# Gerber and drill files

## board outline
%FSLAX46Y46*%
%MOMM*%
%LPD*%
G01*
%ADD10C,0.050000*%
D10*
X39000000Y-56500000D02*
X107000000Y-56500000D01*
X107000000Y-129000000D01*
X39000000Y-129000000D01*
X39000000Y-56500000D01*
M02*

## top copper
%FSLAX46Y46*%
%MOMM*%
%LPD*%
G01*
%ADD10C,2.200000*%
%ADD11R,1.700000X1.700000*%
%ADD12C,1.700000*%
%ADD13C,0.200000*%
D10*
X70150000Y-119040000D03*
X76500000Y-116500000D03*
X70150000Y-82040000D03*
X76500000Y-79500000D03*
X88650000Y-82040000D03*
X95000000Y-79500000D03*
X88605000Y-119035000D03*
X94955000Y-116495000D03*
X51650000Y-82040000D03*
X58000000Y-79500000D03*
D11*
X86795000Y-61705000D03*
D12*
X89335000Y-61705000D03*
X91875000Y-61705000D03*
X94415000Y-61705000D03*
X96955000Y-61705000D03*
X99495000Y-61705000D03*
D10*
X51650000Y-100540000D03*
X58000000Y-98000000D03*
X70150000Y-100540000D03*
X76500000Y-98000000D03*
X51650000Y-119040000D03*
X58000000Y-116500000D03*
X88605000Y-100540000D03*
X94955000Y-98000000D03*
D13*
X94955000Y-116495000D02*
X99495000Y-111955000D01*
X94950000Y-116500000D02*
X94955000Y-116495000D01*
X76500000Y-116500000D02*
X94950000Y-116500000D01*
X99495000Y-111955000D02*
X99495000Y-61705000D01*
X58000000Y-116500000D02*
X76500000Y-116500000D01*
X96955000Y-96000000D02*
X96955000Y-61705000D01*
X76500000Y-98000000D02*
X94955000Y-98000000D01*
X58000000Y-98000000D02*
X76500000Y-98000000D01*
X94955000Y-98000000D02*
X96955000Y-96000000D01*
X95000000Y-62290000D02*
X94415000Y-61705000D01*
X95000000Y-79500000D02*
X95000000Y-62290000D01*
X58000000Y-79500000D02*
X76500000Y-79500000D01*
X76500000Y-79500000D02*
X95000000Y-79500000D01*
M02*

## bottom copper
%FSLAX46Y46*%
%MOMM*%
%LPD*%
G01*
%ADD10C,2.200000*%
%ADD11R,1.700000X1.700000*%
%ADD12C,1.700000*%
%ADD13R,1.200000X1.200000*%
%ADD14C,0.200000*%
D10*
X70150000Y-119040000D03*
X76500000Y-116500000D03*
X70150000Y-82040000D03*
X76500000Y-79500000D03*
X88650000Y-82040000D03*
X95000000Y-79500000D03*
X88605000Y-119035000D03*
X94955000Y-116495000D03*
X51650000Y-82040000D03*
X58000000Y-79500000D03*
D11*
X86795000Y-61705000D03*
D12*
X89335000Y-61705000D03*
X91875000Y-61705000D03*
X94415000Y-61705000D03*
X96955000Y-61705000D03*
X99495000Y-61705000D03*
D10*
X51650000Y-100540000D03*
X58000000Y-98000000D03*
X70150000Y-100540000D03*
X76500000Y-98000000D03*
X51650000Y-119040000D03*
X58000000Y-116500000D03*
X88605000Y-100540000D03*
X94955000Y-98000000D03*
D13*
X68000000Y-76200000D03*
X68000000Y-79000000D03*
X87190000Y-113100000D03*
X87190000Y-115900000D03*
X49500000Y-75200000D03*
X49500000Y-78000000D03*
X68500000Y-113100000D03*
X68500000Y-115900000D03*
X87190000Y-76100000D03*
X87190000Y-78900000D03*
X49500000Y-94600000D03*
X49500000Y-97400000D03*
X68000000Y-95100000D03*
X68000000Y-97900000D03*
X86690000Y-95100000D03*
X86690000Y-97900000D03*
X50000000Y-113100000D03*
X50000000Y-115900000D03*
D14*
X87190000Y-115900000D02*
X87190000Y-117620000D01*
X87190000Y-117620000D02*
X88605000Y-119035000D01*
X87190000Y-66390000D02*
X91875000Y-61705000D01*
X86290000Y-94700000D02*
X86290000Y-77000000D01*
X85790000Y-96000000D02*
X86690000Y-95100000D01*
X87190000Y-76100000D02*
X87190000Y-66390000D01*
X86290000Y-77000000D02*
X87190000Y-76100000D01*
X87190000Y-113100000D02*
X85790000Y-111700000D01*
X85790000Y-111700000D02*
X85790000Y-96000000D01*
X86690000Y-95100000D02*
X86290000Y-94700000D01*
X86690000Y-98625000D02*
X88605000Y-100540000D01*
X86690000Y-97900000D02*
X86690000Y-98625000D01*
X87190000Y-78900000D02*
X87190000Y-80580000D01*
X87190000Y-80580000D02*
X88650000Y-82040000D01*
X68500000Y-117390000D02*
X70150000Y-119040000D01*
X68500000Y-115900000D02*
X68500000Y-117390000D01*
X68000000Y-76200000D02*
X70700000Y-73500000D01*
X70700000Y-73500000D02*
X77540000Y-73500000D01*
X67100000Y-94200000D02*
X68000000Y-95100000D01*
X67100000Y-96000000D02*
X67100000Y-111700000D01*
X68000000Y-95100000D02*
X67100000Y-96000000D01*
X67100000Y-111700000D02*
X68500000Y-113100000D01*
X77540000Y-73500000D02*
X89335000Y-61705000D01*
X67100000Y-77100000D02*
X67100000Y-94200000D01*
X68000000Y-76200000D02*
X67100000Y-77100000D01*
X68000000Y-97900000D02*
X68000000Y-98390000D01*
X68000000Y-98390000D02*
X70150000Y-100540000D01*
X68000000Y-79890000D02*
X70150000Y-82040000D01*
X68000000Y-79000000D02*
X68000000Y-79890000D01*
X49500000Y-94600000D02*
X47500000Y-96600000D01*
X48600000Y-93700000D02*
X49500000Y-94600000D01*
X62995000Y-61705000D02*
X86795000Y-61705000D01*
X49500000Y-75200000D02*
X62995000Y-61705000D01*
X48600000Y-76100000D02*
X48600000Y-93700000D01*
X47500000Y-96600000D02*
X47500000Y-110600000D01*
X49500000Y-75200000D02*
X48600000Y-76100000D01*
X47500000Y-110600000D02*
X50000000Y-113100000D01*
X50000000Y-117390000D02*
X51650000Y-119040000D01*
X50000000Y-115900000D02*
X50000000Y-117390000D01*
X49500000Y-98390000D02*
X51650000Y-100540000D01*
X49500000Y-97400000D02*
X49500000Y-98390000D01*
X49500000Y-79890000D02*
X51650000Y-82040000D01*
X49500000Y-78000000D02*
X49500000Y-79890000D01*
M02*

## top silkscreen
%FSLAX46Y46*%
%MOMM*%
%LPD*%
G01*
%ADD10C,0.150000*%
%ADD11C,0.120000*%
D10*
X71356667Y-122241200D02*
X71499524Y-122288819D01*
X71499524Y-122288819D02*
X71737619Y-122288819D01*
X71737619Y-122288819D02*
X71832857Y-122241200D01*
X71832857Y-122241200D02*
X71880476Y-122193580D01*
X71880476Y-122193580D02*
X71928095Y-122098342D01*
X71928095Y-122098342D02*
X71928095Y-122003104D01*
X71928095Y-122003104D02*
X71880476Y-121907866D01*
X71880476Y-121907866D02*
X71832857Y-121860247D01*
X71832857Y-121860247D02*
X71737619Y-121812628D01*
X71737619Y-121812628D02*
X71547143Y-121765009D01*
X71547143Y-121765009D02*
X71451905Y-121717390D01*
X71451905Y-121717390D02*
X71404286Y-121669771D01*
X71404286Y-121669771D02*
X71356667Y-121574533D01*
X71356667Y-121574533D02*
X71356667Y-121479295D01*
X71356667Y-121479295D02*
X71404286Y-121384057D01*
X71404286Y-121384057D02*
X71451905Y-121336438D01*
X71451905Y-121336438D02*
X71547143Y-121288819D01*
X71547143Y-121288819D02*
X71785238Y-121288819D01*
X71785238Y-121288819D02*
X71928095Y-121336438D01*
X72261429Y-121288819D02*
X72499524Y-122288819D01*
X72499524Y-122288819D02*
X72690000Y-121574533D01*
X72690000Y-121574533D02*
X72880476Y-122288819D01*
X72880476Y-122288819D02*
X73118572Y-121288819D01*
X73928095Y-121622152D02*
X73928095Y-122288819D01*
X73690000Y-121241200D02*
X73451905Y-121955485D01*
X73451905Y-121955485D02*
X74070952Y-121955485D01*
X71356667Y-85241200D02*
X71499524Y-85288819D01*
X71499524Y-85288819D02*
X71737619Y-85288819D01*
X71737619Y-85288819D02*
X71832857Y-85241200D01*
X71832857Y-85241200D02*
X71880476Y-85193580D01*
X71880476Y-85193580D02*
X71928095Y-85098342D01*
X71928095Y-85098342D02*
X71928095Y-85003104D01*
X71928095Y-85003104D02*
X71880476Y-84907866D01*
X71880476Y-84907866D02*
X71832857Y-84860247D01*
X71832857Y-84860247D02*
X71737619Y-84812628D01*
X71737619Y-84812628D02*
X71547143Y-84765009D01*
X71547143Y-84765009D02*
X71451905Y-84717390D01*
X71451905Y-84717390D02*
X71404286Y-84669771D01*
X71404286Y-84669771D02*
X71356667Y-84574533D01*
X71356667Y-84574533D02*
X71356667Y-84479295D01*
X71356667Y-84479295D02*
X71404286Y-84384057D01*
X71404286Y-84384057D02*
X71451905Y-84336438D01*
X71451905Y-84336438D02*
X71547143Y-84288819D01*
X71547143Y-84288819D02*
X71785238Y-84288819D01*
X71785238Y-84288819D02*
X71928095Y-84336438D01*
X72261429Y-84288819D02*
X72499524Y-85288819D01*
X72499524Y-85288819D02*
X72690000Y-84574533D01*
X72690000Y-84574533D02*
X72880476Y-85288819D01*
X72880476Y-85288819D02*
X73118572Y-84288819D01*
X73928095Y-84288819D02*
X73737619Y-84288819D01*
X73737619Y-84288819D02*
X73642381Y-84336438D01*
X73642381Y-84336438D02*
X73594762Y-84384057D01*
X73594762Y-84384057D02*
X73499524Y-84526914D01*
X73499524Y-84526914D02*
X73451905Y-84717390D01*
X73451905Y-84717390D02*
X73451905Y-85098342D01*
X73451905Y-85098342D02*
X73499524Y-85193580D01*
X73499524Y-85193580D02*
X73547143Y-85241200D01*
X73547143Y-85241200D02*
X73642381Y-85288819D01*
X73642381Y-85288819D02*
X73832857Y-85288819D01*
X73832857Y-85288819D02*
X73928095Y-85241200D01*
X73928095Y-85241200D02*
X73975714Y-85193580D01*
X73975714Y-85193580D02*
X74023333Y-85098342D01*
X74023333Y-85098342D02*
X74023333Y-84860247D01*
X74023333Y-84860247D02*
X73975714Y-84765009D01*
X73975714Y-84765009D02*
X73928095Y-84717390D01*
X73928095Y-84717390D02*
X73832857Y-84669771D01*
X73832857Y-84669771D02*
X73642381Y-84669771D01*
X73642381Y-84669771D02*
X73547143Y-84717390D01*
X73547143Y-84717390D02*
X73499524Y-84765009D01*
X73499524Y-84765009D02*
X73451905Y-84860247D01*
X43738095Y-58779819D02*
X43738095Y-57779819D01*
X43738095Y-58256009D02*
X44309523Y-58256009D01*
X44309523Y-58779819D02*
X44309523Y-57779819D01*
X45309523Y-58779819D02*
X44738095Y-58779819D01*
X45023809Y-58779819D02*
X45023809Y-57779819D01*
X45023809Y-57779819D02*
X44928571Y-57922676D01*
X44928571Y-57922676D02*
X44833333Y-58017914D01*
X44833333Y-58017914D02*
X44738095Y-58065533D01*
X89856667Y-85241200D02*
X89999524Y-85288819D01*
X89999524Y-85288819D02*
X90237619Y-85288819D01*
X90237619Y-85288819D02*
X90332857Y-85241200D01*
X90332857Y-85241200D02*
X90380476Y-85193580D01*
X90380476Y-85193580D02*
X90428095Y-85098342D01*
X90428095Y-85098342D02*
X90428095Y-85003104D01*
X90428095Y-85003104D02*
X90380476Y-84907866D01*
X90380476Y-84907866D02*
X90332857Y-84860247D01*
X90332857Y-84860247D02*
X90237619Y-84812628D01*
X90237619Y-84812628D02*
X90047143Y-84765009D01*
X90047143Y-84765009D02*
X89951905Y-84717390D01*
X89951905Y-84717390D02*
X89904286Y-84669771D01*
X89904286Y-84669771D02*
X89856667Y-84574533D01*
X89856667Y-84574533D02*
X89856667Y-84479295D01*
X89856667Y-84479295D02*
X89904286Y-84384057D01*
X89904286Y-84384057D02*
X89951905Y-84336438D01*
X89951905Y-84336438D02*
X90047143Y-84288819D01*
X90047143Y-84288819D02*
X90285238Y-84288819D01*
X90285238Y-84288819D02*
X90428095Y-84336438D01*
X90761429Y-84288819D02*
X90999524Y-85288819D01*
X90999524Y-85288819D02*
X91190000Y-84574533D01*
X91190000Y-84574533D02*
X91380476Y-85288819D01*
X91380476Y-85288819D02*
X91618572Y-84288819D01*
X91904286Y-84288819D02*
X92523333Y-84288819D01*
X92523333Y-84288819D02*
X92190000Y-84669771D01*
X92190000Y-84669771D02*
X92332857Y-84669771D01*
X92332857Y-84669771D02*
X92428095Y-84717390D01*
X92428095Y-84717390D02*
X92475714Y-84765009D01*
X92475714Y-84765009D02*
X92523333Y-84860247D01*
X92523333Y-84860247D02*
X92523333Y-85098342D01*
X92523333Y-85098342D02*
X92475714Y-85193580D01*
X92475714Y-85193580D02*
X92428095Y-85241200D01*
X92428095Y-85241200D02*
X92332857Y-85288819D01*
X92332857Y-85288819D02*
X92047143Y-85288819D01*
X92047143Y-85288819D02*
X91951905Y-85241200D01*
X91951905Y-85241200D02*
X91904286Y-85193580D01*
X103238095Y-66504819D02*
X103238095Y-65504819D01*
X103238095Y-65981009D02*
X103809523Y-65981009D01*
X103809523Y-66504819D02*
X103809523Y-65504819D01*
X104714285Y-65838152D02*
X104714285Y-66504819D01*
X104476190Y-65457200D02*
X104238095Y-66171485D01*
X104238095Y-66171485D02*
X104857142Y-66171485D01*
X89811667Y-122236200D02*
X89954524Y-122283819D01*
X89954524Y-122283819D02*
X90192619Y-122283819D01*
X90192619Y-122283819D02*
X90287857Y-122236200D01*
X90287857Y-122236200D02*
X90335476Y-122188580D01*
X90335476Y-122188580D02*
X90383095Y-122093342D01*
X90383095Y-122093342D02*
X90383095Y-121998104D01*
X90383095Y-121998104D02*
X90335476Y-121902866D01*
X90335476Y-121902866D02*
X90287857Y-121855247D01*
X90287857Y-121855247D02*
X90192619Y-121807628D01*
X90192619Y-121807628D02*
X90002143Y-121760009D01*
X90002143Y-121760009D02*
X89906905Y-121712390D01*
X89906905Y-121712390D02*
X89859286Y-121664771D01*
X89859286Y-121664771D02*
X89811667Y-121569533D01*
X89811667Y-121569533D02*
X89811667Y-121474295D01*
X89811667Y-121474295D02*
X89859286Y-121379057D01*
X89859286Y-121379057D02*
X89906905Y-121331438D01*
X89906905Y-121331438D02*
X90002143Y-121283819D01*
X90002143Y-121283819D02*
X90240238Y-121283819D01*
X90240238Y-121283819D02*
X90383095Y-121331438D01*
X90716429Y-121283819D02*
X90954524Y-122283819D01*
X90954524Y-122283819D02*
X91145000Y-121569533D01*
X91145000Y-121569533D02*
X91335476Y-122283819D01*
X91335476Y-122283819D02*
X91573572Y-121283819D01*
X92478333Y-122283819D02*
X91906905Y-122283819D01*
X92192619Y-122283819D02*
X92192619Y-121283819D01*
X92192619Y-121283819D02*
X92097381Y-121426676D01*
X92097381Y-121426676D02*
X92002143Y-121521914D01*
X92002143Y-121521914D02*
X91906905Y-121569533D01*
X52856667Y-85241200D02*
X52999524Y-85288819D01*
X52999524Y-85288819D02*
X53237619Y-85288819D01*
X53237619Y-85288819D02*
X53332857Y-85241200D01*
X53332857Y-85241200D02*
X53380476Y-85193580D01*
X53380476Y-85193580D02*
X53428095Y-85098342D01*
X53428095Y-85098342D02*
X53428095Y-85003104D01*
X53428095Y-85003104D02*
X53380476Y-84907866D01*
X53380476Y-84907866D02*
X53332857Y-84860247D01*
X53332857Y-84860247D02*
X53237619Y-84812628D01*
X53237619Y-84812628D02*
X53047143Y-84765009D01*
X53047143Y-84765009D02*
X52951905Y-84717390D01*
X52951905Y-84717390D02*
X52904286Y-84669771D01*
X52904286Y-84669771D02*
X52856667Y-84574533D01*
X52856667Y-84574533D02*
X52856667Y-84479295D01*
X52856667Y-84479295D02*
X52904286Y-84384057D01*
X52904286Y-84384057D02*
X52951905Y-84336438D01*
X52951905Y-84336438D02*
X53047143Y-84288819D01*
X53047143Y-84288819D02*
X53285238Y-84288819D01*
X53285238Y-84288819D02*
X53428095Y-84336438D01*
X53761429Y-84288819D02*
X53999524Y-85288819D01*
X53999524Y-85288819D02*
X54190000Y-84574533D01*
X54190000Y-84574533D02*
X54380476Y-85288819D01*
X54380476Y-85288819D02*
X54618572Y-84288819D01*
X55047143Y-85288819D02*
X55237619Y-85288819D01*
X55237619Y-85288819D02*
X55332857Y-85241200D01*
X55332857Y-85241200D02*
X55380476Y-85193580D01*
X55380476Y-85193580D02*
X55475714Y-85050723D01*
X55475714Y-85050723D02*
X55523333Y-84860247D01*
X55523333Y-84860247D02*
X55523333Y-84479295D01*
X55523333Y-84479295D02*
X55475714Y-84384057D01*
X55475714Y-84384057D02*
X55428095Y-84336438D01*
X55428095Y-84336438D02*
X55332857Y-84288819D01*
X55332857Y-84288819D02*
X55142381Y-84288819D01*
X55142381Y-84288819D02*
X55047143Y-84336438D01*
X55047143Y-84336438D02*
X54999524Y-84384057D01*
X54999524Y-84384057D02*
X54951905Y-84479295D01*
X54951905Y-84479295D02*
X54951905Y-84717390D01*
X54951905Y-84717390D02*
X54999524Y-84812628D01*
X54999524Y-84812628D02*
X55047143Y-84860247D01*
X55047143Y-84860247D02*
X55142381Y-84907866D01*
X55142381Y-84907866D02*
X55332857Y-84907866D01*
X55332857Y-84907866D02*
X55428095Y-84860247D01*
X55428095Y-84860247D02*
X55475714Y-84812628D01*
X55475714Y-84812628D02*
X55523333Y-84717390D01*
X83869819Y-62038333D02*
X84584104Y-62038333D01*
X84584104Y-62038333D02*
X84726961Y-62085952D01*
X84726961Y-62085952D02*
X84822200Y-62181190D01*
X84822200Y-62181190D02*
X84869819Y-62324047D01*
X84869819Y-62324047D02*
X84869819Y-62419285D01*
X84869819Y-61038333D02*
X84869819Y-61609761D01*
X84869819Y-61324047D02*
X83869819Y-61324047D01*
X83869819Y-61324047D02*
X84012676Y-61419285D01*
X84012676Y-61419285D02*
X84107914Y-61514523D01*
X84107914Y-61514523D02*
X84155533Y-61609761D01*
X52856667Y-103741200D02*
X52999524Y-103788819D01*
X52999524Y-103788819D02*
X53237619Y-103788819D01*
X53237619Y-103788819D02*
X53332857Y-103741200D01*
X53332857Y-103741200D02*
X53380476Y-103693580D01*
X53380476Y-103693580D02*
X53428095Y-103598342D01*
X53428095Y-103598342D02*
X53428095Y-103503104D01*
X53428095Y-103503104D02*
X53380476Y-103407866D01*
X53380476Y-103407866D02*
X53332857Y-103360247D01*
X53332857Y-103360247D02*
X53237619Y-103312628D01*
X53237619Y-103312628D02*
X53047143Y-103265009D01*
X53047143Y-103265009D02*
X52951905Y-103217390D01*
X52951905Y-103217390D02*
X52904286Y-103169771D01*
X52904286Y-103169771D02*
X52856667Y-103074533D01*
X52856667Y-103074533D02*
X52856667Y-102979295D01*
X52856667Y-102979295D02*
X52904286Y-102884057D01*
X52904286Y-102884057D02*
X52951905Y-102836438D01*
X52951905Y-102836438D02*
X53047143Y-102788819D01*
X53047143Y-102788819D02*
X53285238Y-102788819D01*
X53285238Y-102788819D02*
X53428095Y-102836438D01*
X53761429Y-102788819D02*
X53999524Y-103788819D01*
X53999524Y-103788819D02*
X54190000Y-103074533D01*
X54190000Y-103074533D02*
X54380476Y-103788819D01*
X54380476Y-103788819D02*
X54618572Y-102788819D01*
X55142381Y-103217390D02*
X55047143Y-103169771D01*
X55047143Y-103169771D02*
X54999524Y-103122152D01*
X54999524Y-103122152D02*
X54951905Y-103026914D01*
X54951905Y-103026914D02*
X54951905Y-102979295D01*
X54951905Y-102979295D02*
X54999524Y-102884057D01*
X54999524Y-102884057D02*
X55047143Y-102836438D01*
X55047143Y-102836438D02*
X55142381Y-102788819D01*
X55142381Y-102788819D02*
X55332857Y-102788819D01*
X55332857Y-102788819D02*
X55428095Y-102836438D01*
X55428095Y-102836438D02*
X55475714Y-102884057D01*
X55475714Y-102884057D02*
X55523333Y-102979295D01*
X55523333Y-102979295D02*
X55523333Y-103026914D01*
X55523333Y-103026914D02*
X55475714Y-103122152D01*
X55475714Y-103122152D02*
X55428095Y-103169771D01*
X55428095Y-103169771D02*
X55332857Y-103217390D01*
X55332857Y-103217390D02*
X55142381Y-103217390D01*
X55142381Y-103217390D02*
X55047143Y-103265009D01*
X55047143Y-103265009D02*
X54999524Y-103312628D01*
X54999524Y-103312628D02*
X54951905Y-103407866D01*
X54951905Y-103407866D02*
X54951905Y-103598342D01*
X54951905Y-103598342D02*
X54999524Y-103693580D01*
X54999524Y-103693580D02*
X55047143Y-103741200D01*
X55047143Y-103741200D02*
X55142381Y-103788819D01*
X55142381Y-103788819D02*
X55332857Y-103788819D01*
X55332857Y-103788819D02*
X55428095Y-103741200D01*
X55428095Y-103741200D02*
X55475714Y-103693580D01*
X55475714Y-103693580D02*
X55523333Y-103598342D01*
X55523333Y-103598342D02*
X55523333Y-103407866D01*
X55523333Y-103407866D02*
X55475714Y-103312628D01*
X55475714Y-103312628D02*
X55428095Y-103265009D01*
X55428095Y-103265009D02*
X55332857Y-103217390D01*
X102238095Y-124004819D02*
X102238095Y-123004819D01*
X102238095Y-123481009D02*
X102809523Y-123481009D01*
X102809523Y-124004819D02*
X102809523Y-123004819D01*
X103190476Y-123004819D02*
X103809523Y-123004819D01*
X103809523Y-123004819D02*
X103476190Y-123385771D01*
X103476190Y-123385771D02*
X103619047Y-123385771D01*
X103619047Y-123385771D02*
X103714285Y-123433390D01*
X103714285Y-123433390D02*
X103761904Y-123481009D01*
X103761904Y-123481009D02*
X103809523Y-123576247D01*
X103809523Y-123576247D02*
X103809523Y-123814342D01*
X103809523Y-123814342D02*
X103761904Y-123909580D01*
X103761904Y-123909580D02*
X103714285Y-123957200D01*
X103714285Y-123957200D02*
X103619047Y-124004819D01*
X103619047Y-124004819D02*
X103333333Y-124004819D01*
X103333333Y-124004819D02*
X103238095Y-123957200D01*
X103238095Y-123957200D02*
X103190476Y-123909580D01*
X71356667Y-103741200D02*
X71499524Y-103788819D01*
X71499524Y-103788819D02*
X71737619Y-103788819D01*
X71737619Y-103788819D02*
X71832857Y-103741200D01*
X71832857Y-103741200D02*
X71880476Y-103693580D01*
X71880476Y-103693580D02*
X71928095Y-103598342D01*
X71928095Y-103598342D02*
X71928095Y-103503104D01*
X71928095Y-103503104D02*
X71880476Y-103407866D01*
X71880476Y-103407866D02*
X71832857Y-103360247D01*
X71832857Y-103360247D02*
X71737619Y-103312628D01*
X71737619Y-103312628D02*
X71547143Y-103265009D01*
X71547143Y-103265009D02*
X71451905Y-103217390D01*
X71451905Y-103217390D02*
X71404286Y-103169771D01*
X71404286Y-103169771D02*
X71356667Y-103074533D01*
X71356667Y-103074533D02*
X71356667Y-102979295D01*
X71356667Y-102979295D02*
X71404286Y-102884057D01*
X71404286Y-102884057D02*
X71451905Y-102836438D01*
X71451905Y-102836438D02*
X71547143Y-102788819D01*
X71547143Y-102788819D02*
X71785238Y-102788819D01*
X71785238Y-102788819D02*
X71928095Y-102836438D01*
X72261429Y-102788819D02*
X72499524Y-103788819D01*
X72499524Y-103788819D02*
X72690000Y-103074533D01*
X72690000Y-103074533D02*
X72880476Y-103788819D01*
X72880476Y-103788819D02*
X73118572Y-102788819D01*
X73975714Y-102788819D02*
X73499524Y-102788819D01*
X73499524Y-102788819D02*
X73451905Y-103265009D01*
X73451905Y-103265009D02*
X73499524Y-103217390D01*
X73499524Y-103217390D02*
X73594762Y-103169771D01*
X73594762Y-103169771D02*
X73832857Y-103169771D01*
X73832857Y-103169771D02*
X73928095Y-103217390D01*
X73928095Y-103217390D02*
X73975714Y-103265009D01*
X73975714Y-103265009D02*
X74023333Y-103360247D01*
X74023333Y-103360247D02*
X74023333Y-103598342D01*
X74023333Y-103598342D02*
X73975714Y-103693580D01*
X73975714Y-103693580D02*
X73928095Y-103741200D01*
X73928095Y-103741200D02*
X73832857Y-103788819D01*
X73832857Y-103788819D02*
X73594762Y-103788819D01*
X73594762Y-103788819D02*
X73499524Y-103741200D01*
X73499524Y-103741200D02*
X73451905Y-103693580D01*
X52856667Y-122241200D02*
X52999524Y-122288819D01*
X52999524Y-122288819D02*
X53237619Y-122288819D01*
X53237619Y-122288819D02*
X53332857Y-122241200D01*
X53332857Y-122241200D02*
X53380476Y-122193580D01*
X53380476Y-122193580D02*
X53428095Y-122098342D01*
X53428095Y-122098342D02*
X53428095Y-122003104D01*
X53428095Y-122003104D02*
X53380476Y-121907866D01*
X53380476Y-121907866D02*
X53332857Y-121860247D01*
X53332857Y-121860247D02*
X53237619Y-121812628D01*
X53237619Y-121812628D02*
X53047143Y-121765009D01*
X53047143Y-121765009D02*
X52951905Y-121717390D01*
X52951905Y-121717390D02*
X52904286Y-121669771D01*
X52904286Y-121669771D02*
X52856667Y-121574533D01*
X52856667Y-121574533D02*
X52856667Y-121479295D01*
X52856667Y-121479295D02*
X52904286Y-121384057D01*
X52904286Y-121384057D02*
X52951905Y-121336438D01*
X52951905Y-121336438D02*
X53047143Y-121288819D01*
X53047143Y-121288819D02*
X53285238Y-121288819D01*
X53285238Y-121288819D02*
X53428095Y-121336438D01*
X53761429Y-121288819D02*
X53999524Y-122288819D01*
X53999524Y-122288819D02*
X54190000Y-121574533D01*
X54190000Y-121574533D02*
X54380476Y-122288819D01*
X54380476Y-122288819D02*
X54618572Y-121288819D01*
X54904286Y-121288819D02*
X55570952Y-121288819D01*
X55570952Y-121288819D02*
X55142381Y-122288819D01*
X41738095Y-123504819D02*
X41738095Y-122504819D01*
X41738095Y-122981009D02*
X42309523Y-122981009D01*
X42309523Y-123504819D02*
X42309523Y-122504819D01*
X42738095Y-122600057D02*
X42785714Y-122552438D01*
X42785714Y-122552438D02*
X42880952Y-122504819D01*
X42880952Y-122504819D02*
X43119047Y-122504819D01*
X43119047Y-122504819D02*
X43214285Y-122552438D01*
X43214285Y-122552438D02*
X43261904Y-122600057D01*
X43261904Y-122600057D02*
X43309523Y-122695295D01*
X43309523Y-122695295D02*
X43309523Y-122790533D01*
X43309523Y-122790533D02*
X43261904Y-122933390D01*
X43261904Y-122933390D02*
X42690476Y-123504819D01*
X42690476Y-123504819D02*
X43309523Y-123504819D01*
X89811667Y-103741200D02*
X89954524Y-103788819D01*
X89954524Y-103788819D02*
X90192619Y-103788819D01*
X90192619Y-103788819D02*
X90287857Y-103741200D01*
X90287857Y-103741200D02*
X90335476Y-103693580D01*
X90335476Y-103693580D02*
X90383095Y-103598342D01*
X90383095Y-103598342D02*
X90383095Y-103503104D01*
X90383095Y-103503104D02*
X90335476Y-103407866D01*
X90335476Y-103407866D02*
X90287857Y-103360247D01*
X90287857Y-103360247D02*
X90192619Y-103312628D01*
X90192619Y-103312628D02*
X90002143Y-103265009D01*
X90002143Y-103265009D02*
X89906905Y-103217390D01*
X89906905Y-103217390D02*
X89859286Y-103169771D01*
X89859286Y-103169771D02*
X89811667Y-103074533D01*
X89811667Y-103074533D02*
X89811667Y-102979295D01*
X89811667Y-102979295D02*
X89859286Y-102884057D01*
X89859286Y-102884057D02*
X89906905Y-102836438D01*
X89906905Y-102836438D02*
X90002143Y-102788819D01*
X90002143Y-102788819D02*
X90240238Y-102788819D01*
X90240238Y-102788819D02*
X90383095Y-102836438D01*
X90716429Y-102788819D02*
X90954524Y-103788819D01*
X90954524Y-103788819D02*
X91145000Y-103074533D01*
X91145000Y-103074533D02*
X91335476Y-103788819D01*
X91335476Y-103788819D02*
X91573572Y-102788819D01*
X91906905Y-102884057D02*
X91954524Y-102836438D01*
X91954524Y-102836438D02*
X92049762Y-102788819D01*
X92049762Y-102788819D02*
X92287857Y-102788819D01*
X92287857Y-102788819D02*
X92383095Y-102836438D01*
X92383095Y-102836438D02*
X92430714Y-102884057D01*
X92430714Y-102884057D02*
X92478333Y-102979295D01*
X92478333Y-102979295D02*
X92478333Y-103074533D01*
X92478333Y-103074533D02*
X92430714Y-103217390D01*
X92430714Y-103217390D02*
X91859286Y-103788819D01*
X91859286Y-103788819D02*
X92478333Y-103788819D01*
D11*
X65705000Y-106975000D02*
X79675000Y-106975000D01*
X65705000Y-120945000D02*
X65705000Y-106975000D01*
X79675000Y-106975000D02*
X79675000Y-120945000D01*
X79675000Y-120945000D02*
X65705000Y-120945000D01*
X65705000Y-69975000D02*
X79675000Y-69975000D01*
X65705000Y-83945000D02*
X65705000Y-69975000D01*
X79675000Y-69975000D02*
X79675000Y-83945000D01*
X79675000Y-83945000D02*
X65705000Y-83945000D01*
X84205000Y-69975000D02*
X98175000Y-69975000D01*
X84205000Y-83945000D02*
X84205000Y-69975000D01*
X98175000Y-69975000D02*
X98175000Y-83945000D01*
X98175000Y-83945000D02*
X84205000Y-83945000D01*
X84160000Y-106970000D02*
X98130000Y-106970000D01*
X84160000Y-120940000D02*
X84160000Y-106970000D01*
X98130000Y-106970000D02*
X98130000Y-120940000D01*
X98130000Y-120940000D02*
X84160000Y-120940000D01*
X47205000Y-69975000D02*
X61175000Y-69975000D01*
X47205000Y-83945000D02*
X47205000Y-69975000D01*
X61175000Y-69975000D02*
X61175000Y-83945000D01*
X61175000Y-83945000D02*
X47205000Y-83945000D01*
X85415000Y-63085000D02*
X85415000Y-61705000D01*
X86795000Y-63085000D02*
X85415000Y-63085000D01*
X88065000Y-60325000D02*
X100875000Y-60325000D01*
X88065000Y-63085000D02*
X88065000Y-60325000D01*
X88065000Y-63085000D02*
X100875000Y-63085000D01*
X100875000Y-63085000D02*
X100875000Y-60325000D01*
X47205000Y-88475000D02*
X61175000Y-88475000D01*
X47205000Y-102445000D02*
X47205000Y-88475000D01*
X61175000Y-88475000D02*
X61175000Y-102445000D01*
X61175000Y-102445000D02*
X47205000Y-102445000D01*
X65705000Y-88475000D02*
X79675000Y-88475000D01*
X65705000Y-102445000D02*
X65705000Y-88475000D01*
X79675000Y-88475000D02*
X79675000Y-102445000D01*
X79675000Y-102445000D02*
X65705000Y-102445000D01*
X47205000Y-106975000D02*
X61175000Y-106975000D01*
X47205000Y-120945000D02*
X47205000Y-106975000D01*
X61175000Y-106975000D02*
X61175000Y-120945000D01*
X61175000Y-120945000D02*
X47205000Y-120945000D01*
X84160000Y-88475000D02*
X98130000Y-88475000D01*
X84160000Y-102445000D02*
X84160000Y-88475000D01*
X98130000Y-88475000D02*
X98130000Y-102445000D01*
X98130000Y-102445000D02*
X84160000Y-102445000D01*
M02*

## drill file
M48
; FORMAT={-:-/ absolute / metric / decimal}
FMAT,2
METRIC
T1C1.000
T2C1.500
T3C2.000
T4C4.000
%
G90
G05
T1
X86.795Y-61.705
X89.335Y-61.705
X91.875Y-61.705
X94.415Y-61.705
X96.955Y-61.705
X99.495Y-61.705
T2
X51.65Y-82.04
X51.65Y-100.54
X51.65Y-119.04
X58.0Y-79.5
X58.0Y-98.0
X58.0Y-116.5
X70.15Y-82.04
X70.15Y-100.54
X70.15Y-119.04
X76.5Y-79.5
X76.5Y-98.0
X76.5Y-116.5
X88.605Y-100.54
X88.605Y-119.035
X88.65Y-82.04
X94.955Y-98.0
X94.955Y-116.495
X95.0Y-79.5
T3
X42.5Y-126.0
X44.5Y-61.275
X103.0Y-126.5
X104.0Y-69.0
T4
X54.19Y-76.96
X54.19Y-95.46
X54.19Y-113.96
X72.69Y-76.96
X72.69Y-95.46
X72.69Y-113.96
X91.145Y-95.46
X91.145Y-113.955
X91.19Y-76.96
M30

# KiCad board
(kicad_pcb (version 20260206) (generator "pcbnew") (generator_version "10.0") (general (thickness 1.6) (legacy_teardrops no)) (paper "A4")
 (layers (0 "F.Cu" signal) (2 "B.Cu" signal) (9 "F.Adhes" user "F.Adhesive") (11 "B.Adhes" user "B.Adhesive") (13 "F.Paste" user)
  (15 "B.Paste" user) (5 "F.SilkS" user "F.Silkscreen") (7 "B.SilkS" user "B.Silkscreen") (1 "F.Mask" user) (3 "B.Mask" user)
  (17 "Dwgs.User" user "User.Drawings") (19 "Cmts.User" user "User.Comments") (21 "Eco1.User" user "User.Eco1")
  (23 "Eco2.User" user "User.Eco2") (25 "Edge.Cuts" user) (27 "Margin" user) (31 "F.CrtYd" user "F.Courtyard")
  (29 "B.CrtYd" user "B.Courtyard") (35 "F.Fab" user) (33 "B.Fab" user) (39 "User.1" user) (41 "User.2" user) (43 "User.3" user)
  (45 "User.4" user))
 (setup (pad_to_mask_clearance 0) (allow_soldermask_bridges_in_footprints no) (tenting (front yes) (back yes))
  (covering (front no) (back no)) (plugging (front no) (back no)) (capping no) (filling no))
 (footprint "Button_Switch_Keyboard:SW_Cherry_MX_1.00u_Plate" (layer "F.Cu") (at 70.15 119.04 180)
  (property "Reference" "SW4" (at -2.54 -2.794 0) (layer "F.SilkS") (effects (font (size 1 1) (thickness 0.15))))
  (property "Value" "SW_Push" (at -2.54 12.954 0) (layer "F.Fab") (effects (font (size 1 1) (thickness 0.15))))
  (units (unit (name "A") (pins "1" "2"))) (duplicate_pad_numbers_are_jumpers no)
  (fp_line (start 4.445 12.065) (end -9.525 12.065) (stroke (width 0.12) (type solid)) (layer "F.SilkS"))
  (fp_line (start 4.445 -1.905) (end 4.445 12.065) (stroke (width 0.12) (type solid)) (layer "F.SilkS"))
  (fp_line (start -9.525 12.065) (end -9.525 -1.905) (stroke (width 0.12) (type solid)) (layer "F.SilkS"))
  (fp_line (start -9.525 -1.905) (end 4.445 -1.905) (stroke (width 0.12) (type solid)) (layer "F.SilkS"))
  (pad "" np_thru_hole circle (at -2.54 5.08 180) (size 4 4) (drill 4) (layers "*.Cu" "*.Mask"))
  (pad "1" thru_hole circle (at 0 0 180) (size 2.2 2.2) (drill 1.5) (layers "*.Cu" "*.Mask") (remove_unused_layers no) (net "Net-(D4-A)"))
  (pad "2" thru_hole circle (at -6.35 2.54 180) (size 2.2 2.2) (drill 1.5) (layers "*.Cu" "*.Mask") (remove_unused_layers no) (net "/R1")))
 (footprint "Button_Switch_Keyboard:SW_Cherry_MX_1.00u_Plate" (layer "F.Cu") (at 70.15 82.04 180)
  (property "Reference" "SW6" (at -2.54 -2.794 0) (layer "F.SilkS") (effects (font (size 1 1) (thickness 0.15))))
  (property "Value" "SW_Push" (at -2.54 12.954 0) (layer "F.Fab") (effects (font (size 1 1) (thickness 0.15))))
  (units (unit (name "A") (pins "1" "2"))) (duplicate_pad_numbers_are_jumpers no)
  (fp_line (start 4.445 12.065) (end -9.525 12.065) (stroke (width 0.12) (type solid)) (layer "F.SilkS"))
  (fp_line (start 4.445 -1.905) (end 4.445 12.065) (stroke (width 0.12) (type solid)) (layer "F.SilkS"))
  (fp_line (start -9.525 12.065) (end -9.525 -1.905) (stroke (width 0.12) (type solid)) (layer "F.SilkS"))
  (fp_line (start -9.525 -1.905) (end 4.445 -1.905) (stroke (width 0.12) (type solid)) (layer "F.SilkS"))
  (pad "" np_thru_hole circle (at -2.54 5.08 180) (size 4 4) (drill 4) (layers "*.Cu" "*.Mask"))
  (pad "1" thru_hole circle (at 0 0 180) (size 2.2 2.2) (drill 1.5) (layers "*.Cu" "*.Mask") (remove_unused_layers no) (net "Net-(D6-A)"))
  (pad "2" thru_hole circle (at -6.35 2.54 180) (size 2.2 2.2) (drill 1.5) (layers "*.Cu" "*.Mask") (remove_unused_layers no) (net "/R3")))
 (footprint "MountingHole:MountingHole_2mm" (layer "F.Cu") (at 44.5 61.275)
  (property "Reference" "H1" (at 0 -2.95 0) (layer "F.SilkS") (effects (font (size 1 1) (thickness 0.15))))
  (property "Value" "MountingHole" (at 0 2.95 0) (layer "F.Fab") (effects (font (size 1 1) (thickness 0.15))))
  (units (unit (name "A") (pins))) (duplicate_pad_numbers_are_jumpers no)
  (pad "" np_thru_hole circle (at 0 0) (size 2 2) (drill 2) (layers "*.Cu" "*.Mask")))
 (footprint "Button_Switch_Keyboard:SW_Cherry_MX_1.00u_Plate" (layer "F.Cu") (at 88.65 82.04 180)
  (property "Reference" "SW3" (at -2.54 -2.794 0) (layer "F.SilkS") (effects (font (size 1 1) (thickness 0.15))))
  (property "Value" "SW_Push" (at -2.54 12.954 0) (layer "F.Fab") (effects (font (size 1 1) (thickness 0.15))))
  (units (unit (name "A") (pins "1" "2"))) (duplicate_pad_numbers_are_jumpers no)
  (fp_line (start 4.445 12.065) (end -9.525 12.065) (stroke (width 0.12) (type solid)) (layer "F.SilkS"))
  (fp_line (start 4.445 -1.905) (end 4.445 12.065) (stroke (width 0.12) (type solid)) (layer "F.SilkS"))
  (fp_line (start -9.525 12.065) (end -9.525 -1.905) (stroke (width 0.12) (type solid)) (layer "F.SilkS"))
  (fp_line (start -9.525 -1.905) (end 4.445 -1.905) (stroke (width 0.12) (type solid)) (layer "F.SilkS"))
  (pad "" np_thru_hole circle (at -2.54 5.08 180) (size 4 4) (drill 4) (layers "*.Cu" "*.Mask"))
  (pad "1" thru_hole circle (at 0 0 180) (size 2.2 2.2) (drill 1.5) (layers "*.Cu" "*.Mask") (remove_unused_layers no) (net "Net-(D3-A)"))
  (pad "2" thru_hole circle (at -6.35 2.54 180) (size 2.2 2.2) (drill 1.5) (layers "*.Cu" "*.Mask") (remove_unused_layers no) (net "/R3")))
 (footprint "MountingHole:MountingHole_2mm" (layer "F.Cu") (at 104 69)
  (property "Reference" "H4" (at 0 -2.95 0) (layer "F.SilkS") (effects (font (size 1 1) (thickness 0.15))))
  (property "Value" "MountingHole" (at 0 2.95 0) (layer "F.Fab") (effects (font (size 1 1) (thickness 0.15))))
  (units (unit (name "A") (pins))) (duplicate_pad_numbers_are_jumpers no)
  (pad "" np_thru_hole circle (at 0 0) (size 2 2) (drill 2) (layers "*.Cu" "*.Mask")))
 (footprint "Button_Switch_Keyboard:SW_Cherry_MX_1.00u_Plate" (layer "F.Cu") (at 88.605 119.035 180)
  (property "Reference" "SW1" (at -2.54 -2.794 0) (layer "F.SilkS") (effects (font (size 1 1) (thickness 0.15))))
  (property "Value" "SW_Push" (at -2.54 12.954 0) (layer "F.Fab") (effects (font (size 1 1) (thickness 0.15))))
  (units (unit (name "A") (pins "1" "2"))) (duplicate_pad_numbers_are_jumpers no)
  (fp_line (start 4.445 12.065) (end -9.525 12.065) (stroke (width 0.12) (type solid)) (layer "F.SilkS"))
  (fp_line (start 4.445 -1.905) (end 4.445 12.065) (stroke (width 0.12) (type solid)) (layer "F.SilkS"))
  (fp_line (start -9.525 12.065) (end -9.525 -1.905) (stroke (width 0.12) (type solid)) (layer "F.SilkS"))
  (fp_line (start -9.525 -1.905) (end 4.445 -1.905) (stroke (width 0.12) (type solid)) (layer "F.SilkS"))
  (pad "" np_thru_hole circle (at -2.54 5.08 180) (size 4 4) (drill 4) (layers "*.Cu" "*.Mask"))
  (pad "1" thru_hole circle (at 0 0 180) (size 2.2 2.2) (drill 1.5) (layers "*.Cu" "*.Mask") (remove_unused_layers no) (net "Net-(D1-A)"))
  (pad "2" thru_hole circle (at -6.35 2.54 180) (size 2.2 2.2) (drill 1.5) (layers "*.Cu" "*.Mask") (remove_unused_layers no) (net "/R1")))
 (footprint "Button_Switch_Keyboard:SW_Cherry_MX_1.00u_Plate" (layer "F.Cu") (at 51.65 82.04 180)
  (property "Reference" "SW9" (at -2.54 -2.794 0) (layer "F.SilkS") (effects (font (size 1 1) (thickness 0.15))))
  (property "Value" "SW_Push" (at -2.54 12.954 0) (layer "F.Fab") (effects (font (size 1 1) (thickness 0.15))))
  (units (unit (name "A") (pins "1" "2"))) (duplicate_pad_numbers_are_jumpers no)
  (fp_line (start 4.445 12.065) (end -9.525 12.065) (stroke (width 0.12) (type solid)) (layer "F.SilkS"))
  (fp_line (start 4.445 -1.905) (end 4.445 12.065) (stroke (width 0.12) (type solid)) (layer "F.SilkS"))
  (fp_line (start -9.525 12.065) (end -9.525 -1.905) (stroke (width 0.12) (type solid)) (layer "F.SilkS"))
  (fp_line (start -9.525 -1.905) (end 4.445 -1.905) (stroke (width 0.12) (type solid)) (layer "F.SilkS"))
  (pad "" np_thru_hole circle (at -2.54 5.08 180) (size 4 4) (drill 4) (layers "*.Cu" "*.Mask"))
  (pad "1" thru_hole circle (at 0 0 180) (size 2.2 2.2) (drill 1.5) (layers "*.Cu" "*.Mask") (remove_unused_layers no) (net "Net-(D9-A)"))
  (pad "2" thru_hole circle (at -6.35 2.54 180) (size 2.2 2.2) (drill 1.5) (layers "*.Cu" "*.Mask") (remove_unused_layers no) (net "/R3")))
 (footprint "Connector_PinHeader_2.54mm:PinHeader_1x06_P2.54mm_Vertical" (layer "F.Cu") (at 86.795 61.705 90)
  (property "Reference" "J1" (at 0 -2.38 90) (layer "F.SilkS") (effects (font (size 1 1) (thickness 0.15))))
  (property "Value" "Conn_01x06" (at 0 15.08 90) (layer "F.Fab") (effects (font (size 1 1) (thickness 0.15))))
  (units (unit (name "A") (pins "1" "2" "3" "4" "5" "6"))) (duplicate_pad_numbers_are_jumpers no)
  (fp_line (start -1.38 -1.38) (end 0 -1.38) (stroke (width 0.12) (type solid)) (layer "F.SilkS"))
  (fp_line (start -1.38 0) (end -1.38 -1.38) (stroke (width 0.12) (type solid)) (layer "F.SilkS"))
  (fp_line (start 1.38 1.27) (end 1.38 14.08) (stroke (width 0.12) (type solid)) (layer "F.SilkS"))
  (fp_line (start -1.38 1.27) (end 1.38 1.27) (stroke (width 0.12) (type solid)) (layer "F.SilkS"))
  (fp_line (start -1.38 1.27) (end -1.38 14.08) (stroke (width 0.12) (type solid)) (layer "F.SilkS"))
  (fp_line (start -1.38 14.08) (end 1.38 14.08) (stroke (width 0.12) (type solid)) (layer "F.SilkS"))
  (pad "1" thru_hole rect (at 0 0 90) (size 1.7 1.7) (drill 1) (layers "*.Cu" "*.Mask") (remove_unused_layers no) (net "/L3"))
  (pad "2" thru_hole circle (at 0 2.54 90) (size 1.7 1.7) (drill 1) (layers "*.Cu" "*.Mask") (remove_unused_layers no) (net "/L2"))
  (pad "3" thru_hole circle (at 0 5.08 90) (size 1.7 1.7) (drill 1) (layers "*.Cu" "*.Mask") (remove_unused_layers no) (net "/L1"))
  (pad "4" thru_hole circle (at 0 7.62 90) (size 1.7 1.7) (drill 1) (layers "*.Cu" "*.Mask") (remove_unused_layers no) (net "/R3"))
  (pad "5" thru_hole circle (at 0 10.16 90) (size 1.7 1.7) (drill 1) (layers "*.Cu" "*.Mask") (remove_unused_layers no) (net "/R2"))
  (pad "6" thru_hole circle (at 0 12.7 90) (size 1.7 1.7) (drill 1) (layers "*.Cu" "*.Mask") (remove_unused_layers no) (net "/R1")))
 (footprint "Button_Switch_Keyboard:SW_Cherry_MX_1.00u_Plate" (layer "F.Cu") (at 51.65 100.54 180)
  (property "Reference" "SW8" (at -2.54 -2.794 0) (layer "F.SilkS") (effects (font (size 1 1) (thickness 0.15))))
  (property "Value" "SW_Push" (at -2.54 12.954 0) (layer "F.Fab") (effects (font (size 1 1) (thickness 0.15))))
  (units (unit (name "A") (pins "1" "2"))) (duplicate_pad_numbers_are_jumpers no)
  (fp_line (start 4.445 12.065) (end -9.525 12.065) (stroke (width 0.12) (type solid)) (layer "F.SilkS"))
  (fp_line (start 4.445 -1.905) (end 4.445 12.065) (stroke (width 0.12) (type solid)) (layer "F.SilkS"))
  (fp_line (start -9.525 12.065) (end -9.525 -1.905) (stroke (width 0.12) (type solid)) (layer "F.SilkS"))
  (fp_line (start -9.525 -1.905) (end 4.445 -1.905) (stroke (width 0.12) (type solid)) (layer "F.SilkS"))
  (pad "" np_thru_hole circle (at -2.54 5.08 180) (size 4 4) (drill 4) (layers "*.Cu" "*.Mask"))
  (pad "1" thru_hole circle (at 0 0 180) (size 2.2 2.2) (drill 1.5) (layers "*.Cu" "*.Mask") (remove_unused_layers no) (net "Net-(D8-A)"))
  (pad "2" thru_hole circle (at -6.35 2.54 180) (size 2.2 2.2) (drill 1.5) (layers "*.Cu" "*.Mask") (remove_unused_layers no) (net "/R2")))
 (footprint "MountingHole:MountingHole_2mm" (layer "F.Cu") (at 103 126.5)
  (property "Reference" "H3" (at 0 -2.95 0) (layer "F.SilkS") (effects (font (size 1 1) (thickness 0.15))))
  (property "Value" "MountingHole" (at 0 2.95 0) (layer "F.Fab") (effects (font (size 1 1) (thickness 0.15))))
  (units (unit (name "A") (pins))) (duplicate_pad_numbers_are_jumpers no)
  (pad "" np_thru_hole circle (at 0 0) (size 2 2) (drill 2) (layers "*.Cu" "*.Mask")))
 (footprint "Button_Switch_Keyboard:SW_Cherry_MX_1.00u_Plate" (layer "F.Cu") (at 70.15 100.54 180)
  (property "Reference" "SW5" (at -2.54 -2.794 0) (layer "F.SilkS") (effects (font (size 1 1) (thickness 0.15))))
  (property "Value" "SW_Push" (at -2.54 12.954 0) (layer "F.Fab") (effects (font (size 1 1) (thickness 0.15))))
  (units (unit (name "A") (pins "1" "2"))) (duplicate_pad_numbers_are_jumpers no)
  (fp_line (start 4.445 12.065) (end -9.525 12.065) (stroke (width 0.12) (type solid)) (layer "F.SilkS"))
  (fp_line (start 4.445 -1.905) (end 4.445 12.065) (stroke (width 0.12) (type solid)) (layer "F.SilkS"))
  (fp_line (start -9.525 12.065) (end -9.525 -1.905) (stroke (width 0.12) (type solid)) (layer "F.SilkS"))
  (fp_line (start -9.525 -1.905) (end 4.445 -1.905) (stroke (width 0.12) (type solid)) (layer "F.SilkS"))
  (pad "" np_thru_hole circle (at -2.54 5.08 180) (size 4 4) (drill 4) (layers "*.Cu" "*.Mask"))
  (pad "1" thru_hole circle (at 0 0 180) (size 2.2 2.2) (drill 1.5) (layers "*.Cu" "*.Mask") (remove_unused_layers no) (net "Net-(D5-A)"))
  (pad "2" thru_hole circle (at -6.35 2.54 180) (size 2.2 2.2) (drill 1.5) (layers "*.Cu" "*.Mask") (remove_unused_layers no) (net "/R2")))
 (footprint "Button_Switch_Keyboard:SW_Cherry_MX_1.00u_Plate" (layer "F.Cu") (at 51.65 119.04 180)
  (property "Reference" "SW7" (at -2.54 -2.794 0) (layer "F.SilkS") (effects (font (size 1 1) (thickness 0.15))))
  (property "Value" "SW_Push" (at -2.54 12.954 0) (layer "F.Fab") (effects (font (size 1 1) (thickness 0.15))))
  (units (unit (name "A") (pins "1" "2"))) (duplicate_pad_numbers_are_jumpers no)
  (fp_line (start 4.445 12.065) (end -9.525 12.065) (stroke (width 0.12) (type solid)) (layer "F.SilkS"))
  (fp_line (start 4.445 -1.905) (end 4.445 12.065) (stroke (width 0.12) (type solid)) (layer "F.SilkS"))
  (fp_line (start -9.525 12.065) (end -9.525 -1.905) (stroke (width 0.12) (type solid)) (layer "F.SilkS"))
  (fp_line (start -9.525 -1.905) (end 4.445 -1.905) (stroke (width 0.12) (type solid)) (layer "F.SilkS"))
  (pad "" np_thru_hole circle (at -2.54 5.08 180) (size 4 4) (drill 4) (layers "*.Cu" "*.Mask"))
  (pad "1" thru_hole circle (at 0 0 180) (size 2.2 2.2) (drill 1.5) (layers "*.Cu" "*.Mask") (remove_unused_layers no) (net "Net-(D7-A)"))
  (pad "2" thru_hole circle (at -6.35 2.54 180) (size 2.2 2.2) (drill 1.5) (layers "*.Cu" "*.Mask") (remove_unused_layers no) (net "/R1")))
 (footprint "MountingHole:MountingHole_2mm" (layer "F.Cu") (at 42.5 126)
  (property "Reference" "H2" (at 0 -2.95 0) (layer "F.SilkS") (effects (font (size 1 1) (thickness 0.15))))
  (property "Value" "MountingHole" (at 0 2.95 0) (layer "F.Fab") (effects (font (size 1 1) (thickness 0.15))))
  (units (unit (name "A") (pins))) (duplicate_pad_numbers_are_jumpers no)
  (pad "" np_thru_hole circle (at 0 0) (size 2 2) (drill 2) (layers "*.Cu" "*.Mask")))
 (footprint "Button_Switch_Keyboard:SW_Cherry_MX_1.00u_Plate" (layer "F.Cu") (at 88.605 100.54 180)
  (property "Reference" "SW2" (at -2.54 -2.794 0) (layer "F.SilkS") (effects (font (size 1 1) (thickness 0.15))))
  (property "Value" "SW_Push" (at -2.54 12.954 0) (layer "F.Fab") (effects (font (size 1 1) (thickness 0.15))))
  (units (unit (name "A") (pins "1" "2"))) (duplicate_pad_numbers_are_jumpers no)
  (fp_line (start 4.445 12.065) (end -9.525 12.065) (stroke (width 0.12) (type solid)) (layer "F.SilkS"))
  (fp_line (start 4.445 -1.905) (end 4.445 12.065) (stroke (width 0.12) (type solid)) (layer "F.SilkS"))
  (fp_line (start -9.525 12.065) (end -9.525 -1.905) (stroke (width 0.12) (type solid)) (layer "F.SilkS"))
  (fp_line (start -9.525 -1.905) (end 4.445 -1.905) (stroke (width 0.12) (type solid)) (layer "F.SilkS"))
  (pad "" np_thru_hole circle (at -2.54 5.08 180) (size 4 4) (drill 4) (layers "*.Cu" "*.Mask"))
  (pad "1" thru_hole circle (at 0 0 180) (size 2.2 2.2) (drill 1.5) (layers "*.Cu" "*.Mask") (remove_unused_layers no) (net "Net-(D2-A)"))
  (pad "2" thru_hole circle (at -6.35 2.54 180) (size 2.2 2.2) (drill 1.5) (layers "*.Cu" "*.Mask") (remove_unused_layers no) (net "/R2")))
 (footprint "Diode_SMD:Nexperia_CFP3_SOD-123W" (layer "B.Cu") (at 68 77.6 -90)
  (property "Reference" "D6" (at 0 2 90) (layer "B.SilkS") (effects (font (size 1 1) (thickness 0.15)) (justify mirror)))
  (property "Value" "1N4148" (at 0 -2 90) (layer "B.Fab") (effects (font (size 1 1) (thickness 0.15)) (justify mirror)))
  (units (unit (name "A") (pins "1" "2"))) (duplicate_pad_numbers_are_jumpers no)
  (pad "1" smd rect (at -1.4 0 270) (size 1.2 1.2) (layers "B.Cu" "B.Mask" "B.Paste") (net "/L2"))
  (pad "2" smd rect (at 1.4 0 270) (size 1.2 1.2) (layers "B.Cu" "B.Mask" "B.Paste") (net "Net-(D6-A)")))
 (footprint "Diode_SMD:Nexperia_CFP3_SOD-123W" (layer "B.Cu") (at 87.19 114.5 -90)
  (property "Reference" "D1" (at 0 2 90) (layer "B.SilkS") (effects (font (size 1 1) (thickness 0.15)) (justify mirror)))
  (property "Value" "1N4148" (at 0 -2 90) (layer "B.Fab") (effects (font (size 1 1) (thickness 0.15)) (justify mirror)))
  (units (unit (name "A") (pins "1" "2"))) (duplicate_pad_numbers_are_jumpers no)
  (pad "1" smd rect (at -1.4 0 270) (size 1.2 1.2) (layers "B.Cu" "B.Mask" "B.Paste") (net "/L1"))
  (pad "2" smd rect (at 1.4 0 270) (size 1.2 1.2) (layers "B.Cu" "B.Mask" "B.Paste") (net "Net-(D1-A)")))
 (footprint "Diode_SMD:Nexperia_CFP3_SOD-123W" (layer "B.Cu") (at 49.5 76.6 -90)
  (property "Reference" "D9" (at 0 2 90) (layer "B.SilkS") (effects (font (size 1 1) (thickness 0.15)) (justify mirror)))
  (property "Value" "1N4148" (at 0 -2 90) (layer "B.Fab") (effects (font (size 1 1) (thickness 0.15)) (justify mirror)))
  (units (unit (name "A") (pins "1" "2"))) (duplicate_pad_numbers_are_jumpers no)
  (pad "1" smd rect (at -1.4 0 270) (size 1.2 1.2) (layers "B.Cu" "B.Mask" "B.Paste") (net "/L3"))
  (pad "2" smd rect (at 1.4 0 270) (size 1.2 1.2) (layers "B.Cu" "B.Mask" "B.Paste") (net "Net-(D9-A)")))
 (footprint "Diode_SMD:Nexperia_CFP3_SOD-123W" (layer "B.Cu") (at 68.5 114.5 -90)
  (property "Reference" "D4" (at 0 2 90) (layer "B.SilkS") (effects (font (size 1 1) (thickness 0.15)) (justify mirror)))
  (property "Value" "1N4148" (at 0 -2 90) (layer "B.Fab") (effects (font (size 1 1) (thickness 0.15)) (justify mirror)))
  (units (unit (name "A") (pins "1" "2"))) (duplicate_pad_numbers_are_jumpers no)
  (pad "1" smd rect (at -1.4 0 270) (size 1.2 1.2) (layers "B.Cu" "B.Mask" "B.Paste") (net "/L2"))
  (pad "2" smd rect (at 1.4 0 270) (size 1.2 1.2) (layers "B.Cu" "B.Mask" "B.Paste") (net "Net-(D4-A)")))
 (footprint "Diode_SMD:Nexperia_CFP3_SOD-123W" (layer "B.Cu") (at 87.19 77.5 -90)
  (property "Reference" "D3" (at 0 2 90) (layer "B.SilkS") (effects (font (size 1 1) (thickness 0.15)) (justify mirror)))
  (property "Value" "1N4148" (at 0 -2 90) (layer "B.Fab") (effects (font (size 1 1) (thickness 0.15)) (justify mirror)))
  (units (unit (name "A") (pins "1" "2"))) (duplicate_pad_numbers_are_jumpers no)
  (pad "1" smd rect (at -1.4 0 270) (size 1.2 1.2) (layers "B.Cu" "B.Mask" "B.Paste") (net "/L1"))
  (pad "2" smd rect (at 1.4 0 270) (size 1.2 1.2) (layers "B.Cu" "B.Mask" "B.Paste") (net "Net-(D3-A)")))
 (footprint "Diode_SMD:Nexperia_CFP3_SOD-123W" (layer "B.Cu") (at 49.5 96 -90)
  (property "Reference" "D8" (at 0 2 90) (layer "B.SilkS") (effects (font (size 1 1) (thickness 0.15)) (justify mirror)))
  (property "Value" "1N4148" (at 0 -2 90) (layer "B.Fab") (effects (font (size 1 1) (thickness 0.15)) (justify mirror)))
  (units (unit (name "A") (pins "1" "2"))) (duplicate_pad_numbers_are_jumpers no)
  (pad "1" smd rect (at -1.4 0 270) (size 1.2 1.2) (layers "B.Cu" "B.Mask" "B.Paste") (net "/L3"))
  (pad "2" smd rect (at 1.4 0 270) (size 1.2 1.2) (layers "B.Cu" "B.Mask" "B.Paste") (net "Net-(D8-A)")))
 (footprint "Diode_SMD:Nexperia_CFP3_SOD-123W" (layer "B.Cu") (at 68 96.5 -90)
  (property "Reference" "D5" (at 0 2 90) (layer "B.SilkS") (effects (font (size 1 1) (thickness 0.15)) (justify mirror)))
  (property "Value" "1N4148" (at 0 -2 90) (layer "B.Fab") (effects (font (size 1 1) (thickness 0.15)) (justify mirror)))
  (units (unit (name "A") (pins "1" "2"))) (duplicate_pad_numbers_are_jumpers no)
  (pad "1" smd rect (at -1.4 0 270) (size 1.2 1.2) (layers "B.Cu" "B.Mask" "B.Paste") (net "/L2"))
  (pad "2" smd rect (at 1.4 0 270) (size 1.2 1.2) (layers "B.Cu" "B.Mask" "B.Paste") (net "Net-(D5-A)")))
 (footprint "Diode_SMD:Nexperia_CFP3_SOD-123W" (layer "B.Cu") (at 86.69 96.5 -90)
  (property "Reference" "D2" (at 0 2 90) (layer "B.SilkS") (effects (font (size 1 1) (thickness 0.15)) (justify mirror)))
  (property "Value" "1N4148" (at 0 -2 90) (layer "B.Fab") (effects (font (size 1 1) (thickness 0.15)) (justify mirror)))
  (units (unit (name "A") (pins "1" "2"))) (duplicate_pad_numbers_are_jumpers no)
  (pad "1" smd rect (at -1.4 0 270) (size 1.2 1.2) (layers "B.Cu" "B.Mask" "B.Paste") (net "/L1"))
  (pad "2" smd rect (at 1.4 0 270) (size 1.2 1.2) (layers "B.Cu" "B.Mask" "B.Paste") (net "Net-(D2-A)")))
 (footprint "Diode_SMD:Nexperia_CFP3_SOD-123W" (layer "B.Cu") (at 50 114.5 -90)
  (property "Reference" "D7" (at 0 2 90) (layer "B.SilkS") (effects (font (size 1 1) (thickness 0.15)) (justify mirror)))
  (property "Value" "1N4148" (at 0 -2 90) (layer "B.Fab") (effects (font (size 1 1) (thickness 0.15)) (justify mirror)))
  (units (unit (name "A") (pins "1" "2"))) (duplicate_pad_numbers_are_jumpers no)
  (pad "1" smd rect (at -1.4 0 270) (size 1.2 1.2) (layers "B.Cu" "B.Mask" "B.Paste") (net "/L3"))
  (pad "2" smd rect (at 1.4 0 270) (size 1.2 1.2) (layers "B.Cu" "B.Mask" "B.Paste") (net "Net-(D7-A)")))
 (gr_rect (start 39 56.5) (end 107 129) (stroke (width 0.05) (type default)) (fill no) (layer "Edge.Cuts"))
 (segment (start 87.19 115.9) (end 87.19 117.62) (width 0.2) (layer "B.Cu") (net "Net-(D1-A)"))
 (segment (start 87.19 117.62) (end 88.605 119.035) (width 0.2) (layer "B.Cu") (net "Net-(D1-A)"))
 (segment (start 87.19 66.39) (end 91.875 61.705) (width 0.2) (layer "B.Cu") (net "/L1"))
 (segment (start 86.29 94.7) (end 86.29 77) (width 0.2) (layer "B.Cu") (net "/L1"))
 (segment (start 85.79 96) (end 86.69 95.1) (width 0.2) (layer "B.Cu") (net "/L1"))
 (segment (start 87.19 76.1) (end 87.19 66.39) (width 0.2) (layer "B.Cu") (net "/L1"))
 (segment (start 86.29 77) (end 87.19 76.1) (width 0.2) (layer "B.Cu") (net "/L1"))
 (segment (start 87.19 113.1) (end 85.79 111.7) (width 0.2) (layer "B.Cu") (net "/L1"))
 (segment (start 85.79 111.7) (end 85.79 96) (width 0.2) (layer "B.Cu") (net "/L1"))
 (segment (start 86.69 95.1) (end 86.29 94.7) (width 0.2) (layer "B.Cu") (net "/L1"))
 (segment (start 86.69 98.625) (end 88.605 100.54) (width 0.2) (layer "B.Cu") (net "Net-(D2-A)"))
 (segment (start 86.69 97.9) (end 86.69 98.625) (width 0.2) (layer "B.Cu") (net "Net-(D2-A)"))
 (segment (start 87.19 78.9) (end 87.19 80.58) (width 0.2) (layer "B.Cu") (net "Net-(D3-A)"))
 (segment (start 87.19 80.58) (end 88.65 82.04) (width 0.2) (layer "B.Cu") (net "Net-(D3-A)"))
 (segment (start 68.5 117.39) (end 70.15 119.04) (width 0.2) (layer "B.Cu") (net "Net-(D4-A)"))
 (segment (start 68.5 115.9) (end 68.5 117.39) (width 0.2) (layer "B.Cu") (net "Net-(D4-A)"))
 (segment (start 68 76.2) (end 70.7 73.5) (width 0.2) (layer "B.Cu") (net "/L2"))
 (segment (start 70.7 73.5) (end 77.54 73.5) (width 0.2) (layer "B.Cu") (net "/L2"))
 (segment (start 67.1 94.2) (end 68 95.1) (width 0.2) (layer "B.Cu") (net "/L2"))
 (segment (start 67.1 96) (end 67.1 111.7) (width 0.2) (layer "B.Cu") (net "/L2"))
 (segment (start 68 95.1) (end 67.1 96) (width 0.2) (layer "B.Cu") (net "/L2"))
 (segment (start 67.1 111.7) (end 68.5 113.1) (width 0.2) (layer "B.Cu") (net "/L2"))
 (segment (start 77.54 73.5) (end 89.335 61.705) (width 0.2) (layer "B.Cu") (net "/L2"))
 (segment (start 67.1 77.1) (end 67.1 94.2) (width 0.2) (layer "B.Cu") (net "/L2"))
 (segment (start 68 76.2) (end 67.1 77.1) (width 0.2) (layer "B.Cu") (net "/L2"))
 (segment (start 68 97.9) (end 68 98.39) (width 0.2) (layer "B.Cu") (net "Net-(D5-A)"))
 (segment (start 68 98.39) (end 70.15 100.54) (width 0.2) (layer "B.Cu") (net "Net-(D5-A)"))
 (segment (start 68 79.89) (end 70.15 82.04) (width 0.2) (layer "B.Cu") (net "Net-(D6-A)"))
 (segment (start 68 79) (end 68 79.89) (width 0.2) (layer "B.Cu") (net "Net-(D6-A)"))
 (segment (start 49.5 94.6) (end 47.5 96.6) (width 0.2) (layer "B.Cu") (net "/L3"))
 (segment (start 48.6 93.7) (end 49.5 94.6) (width 0.2) (layer "B.Cu") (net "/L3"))
 (segment (start 62.995 61.705) (end 86.795 61.705) (width 0.2) (layer "B.Cu") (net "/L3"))
 (segment (start 49.5 75.2) (end 62.995 61.705) (width 0.2) (layer "B.Cu") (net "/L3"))
 (segment (start 48.6 76.1) (end 48.6 93.7) (width 0.2) (layer "B.Cu") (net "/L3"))
 (segment (start 47.5 96.6) (end 47.5 110.6) (width 0.2) (layer "B.Cu") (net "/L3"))
 (segment (start 49.5 75.2) (end 48.6 76.1) (width 0.2) (layer "B.Cu") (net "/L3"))
 (segment (start 47.5 110.6) (end 50 113.1) (width 0.2) (layer "B.Cu") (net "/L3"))
 (segment (start 50 117.39) (end 51.65 119.04) (width 0.2) (layer "B.Cu") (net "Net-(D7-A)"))
 (segment (start 50 115.9) (end 50 117.39) (width 0.2) (layer "B.Cu") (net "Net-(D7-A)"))
 (segment (start 49.5 98.39) (end 51.65 100.54) (width 0.2) (layer "B.Cu") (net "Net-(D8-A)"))
 (segment (start 49.5 97.4) (end 49.5 98.39) (width 0.2) (layer "B.Cu") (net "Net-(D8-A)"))
 (segment (start 49.5 79.89) (end 51.65 82.04) (width 0.2) (layer "B.Cu") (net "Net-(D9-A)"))
 (segment (start 49.5 78) (end 49.5 79.89) (width 0.2) (layer "B.Cu") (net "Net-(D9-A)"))
 (segment (start 94.955 116.495) (end 99.495 111.955) (width 0.2) (layer "F.Cu") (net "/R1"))
 (segment (start 94.95 116.5) (end 94.955 116.495) (width 0.2) (layer "F.Cu") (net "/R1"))
 (segment (start 76.5 116.5) (end 94.95 116.5) (width 0.2) (layer "F.Cu") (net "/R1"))
 (segment (start 99.495 111.955) (end 99.495 61.705) (width 0.2) (layer "F.Cu") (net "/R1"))
 (segment (start 58 116.5) (end 76.5 116.5) (width 0.2) (layer "F.Cu") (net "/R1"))
 (segment (start 96.955 96) (end 96.955 61.705) (width 0.2) (layer "F.Cu") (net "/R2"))
 (segment (start 76.5 98) (end 94.955 98) (width 0.2) (layer "F.Cu") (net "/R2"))
 (segment (start 58 98) (end 76.5 98) (width 0.2) (layer "F.Cu") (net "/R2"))
 (segment (start 94.955 98) (end 96.955 96) (width 0.2) (layer "F.Cu") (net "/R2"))
 (segment (start 95 62.29) (end 94.415 61.705) (width 0.2) (layer "F.Cu") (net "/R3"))
 (segment (start 95 79.5) (end 95 62.29) (width 0.2) (layer "F.Cu") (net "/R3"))
 (segment (start 58 79.5) (end 76.5 79.5) (width 0.2) (layer "F.Cu") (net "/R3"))
 (segment (start 76.5 79.5) (end 95 79.5) (width 0.2) (layer "F.Cu") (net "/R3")))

